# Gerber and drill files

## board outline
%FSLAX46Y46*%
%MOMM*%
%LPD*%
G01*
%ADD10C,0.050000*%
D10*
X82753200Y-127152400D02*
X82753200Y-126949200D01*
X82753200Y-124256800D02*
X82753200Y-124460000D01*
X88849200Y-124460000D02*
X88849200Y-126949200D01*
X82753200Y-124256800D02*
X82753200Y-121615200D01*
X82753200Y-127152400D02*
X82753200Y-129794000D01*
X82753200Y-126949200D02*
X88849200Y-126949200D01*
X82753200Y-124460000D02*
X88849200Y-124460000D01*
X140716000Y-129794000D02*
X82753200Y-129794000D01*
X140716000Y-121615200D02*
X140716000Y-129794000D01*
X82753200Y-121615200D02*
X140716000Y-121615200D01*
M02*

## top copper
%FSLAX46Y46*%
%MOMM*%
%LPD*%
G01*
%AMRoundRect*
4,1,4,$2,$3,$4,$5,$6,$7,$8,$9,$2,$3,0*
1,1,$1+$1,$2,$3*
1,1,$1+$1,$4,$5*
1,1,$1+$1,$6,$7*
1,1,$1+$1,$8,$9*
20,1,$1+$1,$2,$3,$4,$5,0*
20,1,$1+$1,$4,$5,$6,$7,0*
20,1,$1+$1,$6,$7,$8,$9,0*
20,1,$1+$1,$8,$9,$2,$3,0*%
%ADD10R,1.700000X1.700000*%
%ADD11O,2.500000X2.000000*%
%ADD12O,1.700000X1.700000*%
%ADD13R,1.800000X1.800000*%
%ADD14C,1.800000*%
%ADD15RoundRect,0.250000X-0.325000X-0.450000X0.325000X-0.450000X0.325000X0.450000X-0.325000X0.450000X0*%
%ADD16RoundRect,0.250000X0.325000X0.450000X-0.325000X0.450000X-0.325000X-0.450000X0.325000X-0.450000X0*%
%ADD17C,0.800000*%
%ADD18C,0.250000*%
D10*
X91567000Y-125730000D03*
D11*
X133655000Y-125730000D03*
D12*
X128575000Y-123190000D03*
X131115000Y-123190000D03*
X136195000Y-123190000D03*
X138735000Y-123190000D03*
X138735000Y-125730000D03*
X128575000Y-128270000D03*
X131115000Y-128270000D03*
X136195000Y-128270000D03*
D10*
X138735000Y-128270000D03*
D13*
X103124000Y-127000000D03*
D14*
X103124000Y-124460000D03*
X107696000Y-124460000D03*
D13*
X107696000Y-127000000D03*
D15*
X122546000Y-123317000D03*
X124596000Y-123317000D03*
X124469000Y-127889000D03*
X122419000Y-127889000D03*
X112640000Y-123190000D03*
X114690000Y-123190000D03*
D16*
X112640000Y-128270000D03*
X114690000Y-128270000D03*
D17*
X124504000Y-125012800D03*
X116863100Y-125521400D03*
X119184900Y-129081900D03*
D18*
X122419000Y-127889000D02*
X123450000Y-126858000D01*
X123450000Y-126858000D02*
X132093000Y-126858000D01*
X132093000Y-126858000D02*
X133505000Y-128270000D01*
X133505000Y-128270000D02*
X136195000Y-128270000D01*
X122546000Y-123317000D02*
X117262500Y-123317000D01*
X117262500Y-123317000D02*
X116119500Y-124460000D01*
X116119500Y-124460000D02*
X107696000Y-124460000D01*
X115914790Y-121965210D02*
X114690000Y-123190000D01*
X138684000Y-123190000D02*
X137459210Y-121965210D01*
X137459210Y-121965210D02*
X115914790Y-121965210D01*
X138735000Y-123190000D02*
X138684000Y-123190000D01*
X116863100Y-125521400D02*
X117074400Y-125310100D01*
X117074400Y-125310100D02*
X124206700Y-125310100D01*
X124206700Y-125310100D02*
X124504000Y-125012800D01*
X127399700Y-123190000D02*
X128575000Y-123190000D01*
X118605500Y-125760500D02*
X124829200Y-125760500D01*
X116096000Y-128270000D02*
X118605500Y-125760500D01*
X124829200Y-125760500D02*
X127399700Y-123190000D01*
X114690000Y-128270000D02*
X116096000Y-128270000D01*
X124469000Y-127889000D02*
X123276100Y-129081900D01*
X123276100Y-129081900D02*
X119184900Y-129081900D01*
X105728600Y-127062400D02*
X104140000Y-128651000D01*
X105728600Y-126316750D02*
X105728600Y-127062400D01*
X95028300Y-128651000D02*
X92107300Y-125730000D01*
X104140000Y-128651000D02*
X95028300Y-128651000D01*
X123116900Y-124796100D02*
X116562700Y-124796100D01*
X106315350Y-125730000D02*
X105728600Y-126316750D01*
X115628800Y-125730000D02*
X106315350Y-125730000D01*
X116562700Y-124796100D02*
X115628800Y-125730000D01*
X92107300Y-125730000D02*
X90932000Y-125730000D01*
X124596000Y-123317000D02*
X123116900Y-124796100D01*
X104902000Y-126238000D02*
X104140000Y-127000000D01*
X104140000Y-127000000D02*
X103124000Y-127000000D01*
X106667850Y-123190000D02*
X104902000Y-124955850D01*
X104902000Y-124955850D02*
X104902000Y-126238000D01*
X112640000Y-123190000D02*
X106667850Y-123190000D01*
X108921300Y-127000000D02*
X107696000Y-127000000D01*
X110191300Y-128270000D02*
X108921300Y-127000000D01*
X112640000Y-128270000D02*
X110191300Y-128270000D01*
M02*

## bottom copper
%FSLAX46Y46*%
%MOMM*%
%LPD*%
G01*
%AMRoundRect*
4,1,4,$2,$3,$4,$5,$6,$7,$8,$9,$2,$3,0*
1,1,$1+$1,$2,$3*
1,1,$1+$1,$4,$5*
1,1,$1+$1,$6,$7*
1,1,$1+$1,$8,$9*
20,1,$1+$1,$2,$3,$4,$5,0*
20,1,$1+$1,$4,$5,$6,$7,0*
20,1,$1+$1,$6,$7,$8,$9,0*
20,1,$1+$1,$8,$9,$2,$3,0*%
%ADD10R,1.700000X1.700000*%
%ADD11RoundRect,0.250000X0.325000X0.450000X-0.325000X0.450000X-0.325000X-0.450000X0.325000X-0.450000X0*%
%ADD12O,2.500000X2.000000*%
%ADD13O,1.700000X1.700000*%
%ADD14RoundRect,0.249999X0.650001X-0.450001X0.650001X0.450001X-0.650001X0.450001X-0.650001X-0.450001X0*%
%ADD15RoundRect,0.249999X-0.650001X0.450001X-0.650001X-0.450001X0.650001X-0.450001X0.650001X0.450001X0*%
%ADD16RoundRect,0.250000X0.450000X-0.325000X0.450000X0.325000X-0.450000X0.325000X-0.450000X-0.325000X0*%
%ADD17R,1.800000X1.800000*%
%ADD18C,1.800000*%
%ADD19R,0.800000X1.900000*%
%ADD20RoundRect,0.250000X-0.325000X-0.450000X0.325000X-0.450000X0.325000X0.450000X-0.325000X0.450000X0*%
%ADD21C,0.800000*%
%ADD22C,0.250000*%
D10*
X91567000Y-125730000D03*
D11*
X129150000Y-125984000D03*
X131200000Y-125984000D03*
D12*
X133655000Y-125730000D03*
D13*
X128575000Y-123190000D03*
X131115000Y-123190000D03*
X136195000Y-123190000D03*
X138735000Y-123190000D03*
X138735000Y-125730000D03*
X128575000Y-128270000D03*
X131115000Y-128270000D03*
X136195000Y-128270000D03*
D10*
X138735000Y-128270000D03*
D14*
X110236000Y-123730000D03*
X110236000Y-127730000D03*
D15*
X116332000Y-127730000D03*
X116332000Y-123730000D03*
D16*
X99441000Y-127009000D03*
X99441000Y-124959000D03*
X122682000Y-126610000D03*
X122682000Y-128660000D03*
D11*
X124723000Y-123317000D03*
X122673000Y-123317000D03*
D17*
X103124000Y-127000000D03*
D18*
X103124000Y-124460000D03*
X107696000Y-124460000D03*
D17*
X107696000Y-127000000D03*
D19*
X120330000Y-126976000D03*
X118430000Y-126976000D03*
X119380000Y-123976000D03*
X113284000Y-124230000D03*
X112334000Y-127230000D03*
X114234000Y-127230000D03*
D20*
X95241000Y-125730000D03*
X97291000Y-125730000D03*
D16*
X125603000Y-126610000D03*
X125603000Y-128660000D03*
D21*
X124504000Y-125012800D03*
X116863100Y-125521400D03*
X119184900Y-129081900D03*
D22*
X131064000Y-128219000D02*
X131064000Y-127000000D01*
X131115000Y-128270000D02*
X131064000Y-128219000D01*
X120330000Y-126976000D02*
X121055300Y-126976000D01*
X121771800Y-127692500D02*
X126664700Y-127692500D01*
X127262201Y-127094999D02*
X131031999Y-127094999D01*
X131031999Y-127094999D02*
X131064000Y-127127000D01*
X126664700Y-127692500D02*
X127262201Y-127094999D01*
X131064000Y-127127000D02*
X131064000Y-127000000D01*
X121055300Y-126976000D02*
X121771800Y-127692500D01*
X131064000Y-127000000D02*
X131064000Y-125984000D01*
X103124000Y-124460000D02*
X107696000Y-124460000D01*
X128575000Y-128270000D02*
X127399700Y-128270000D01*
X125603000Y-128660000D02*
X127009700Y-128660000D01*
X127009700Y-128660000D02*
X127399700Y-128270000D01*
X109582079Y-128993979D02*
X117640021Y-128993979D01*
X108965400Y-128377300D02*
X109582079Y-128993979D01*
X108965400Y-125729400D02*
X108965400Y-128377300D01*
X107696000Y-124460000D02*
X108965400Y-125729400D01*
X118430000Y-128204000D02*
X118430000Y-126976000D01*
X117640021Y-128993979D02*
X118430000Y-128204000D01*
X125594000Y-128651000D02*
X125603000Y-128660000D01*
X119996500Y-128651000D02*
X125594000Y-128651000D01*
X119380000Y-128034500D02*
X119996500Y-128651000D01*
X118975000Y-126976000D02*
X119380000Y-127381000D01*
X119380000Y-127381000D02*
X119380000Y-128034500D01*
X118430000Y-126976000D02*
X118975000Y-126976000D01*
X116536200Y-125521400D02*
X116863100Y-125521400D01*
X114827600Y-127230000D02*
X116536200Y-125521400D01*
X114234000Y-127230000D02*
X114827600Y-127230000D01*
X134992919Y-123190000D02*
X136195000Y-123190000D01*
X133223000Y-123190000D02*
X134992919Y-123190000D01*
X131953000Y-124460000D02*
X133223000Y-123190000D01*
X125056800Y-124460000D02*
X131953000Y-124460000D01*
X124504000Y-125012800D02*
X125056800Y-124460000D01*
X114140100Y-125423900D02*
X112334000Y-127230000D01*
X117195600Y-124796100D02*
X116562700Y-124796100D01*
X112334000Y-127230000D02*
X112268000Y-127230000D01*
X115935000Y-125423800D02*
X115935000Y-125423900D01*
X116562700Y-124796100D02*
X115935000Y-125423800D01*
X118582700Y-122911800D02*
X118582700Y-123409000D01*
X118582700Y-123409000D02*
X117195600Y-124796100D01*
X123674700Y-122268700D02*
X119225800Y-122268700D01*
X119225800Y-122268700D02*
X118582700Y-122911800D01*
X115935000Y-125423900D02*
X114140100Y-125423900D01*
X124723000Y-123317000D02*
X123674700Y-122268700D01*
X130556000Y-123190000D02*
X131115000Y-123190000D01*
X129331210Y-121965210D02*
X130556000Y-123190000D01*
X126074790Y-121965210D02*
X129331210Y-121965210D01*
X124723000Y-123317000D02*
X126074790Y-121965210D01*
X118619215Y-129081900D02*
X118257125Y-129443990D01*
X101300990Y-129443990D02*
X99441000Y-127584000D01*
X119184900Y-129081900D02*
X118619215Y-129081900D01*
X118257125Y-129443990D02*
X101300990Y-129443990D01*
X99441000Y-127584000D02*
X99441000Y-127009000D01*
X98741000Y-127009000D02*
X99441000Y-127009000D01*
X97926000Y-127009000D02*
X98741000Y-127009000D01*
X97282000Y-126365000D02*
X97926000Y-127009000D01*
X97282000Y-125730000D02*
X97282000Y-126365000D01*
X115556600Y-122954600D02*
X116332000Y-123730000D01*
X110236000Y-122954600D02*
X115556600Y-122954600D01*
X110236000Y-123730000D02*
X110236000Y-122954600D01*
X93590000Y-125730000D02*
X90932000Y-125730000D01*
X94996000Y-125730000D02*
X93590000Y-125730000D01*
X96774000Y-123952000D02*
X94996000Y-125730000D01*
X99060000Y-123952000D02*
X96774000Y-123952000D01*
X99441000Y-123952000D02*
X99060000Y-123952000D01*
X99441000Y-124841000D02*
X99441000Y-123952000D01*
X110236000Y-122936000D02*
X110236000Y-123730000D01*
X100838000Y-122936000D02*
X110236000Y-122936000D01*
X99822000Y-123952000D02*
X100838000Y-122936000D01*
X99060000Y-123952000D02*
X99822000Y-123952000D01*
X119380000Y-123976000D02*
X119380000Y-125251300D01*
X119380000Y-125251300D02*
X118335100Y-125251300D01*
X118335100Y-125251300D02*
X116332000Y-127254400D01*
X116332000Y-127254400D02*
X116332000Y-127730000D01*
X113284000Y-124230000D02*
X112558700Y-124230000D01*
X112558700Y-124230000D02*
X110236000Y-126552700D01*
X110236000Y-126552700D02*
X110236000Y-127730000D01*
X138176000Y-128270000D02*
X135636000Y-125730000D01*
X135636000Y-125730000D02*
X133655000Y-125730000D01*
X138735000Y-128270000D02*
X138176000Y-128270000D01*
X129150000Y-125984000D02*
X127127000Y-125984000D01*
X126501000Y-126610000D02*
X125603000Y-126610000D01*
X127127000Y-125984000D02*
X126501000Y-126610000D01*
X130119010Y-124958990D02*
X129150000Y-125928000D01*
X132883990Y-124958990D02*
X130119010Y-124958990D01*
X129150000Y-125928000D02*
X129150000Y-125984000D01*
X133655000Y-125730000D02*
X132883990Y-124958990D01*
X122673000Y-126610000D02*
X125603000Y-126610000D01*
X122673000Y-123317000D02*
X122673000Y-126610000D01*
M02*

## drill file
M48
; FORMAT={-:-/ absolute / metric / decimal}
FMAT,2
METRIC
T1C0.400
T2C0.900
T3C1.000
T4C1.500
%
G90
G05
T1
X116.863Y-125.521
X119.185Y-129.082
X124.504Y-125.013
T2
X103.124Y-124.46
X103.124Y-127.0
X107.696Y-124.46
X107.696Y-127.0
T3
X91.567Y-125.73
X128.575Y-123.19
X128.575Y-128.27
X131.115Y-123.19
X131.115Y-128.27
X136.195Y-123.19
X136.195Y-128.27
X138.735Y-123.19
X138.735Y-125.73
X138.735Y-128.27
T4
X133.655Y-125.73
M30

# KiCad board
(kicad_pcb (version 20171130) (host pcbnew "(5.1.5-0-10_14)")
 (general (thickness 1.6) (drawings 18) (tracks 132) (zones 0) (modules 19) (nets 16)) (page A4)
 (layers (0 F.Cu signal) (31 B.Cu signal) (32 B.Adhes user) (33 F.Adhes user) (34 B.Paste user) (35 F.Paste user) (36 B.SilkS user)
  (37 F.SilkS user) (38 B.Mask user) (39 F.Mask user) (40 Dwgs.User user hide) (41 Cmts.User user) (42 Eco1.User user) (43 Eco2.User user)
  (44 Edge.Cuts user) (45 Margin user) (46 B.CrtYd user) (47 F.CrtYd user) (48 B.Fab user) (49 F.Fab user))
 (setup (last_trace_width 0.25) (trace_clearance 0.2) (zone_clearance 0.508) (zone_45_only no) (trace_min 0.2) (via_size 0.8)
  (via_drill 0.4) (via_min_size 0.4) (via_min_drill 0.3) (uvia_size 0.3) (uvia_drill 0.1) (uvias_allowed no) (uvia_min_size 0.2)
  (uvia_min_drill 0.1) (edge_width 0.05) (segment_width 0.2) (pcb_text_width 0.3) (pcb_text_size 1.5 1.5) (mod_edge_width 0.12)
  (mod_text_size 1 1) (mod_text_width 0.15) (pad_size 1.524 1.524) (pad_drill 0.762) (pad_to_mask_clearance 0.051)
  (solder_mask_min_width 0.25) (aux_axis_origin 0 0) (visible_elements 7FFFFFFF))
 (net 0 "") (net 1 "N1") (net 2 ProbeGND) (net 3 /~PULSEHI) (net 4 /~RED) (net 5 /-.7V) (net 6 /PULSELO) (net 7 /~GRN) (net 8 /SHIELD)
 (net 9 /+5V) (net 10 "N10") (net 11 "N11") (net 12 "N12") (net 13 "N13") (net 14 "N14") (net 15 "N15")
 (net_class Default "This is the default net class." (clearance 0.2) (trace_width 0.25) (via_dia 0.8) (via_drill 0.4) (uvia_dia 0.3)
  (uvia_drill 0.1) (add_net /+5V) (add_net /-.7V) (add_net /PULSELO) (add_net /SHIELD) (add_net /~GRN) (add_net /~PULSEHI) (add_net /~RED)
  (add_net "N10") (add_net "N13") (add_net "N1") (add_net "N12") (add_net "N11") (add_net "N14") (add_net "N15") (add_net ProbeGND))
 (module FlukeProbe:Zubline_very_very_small (layer F.Cu) (at 96.774 125.73 60)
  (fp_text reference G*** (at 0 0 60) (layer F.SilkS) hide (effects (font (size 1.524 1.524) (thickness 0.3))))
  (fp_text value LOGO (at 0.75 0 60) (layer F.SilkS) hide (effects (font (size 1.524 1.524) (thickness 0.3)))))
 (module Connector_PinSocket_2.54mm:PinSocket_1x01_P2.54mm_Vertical (layer F.Cu) (at 91.567 125.73)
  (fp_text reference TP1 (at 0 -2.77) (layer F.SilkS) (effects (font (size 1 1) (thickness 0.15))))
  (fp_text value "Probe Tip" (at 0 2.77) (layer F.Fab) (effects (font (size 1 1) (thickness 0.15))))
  (pad 1 thru_hole rect (at 0 0) (size 1.7 1.7) (drill 1) (layers *.Cu *.Mask) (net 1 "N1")))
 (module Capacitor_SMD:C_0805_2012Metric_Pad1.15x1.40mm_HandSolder (layer B.Cu) (at 130.175 125.984 180)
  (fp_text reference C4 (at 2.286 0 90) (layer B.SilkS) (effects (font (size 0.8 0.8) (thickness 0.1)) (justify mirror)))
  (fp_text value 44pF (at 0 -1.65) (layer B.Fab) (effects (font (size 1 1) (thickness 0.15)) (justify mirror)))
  (pad 2 smd roundrect (at 1.025 0 180) (size 1.15 1.4) (layers B.Cu B.Paste B.Mask) (roundrect_rratio 0.217391) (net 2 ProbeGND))
  (pad 1 smd roundrect (at -1.025 0 180) (size 1.15 1.4) (layers B.Cu B.Paste B.Mask) (roundrect_rratio 0.217391) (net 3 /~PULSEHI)))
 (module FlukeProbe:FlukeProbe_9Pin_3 (layer B.Cu) (at 138.735 128.27 90)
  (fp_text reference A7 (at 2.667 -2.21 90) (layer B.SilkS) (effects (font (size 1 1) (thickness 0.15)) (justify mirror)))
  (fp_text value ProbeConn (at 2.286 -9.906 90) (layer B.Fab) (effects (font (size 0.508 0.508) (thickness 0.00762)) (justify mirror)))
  (pad 10 thru_hole oval (at 2.54 -5.08 90) (size 2 2.5) (drill 1.5) (layers *.Cu *.Mask) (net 2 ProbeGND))
  (pad 9 thru_hole oval (at 5.08 -10.16 90) (size 1.7 1.7) (drill 1) (layers *.Cu *.Mask) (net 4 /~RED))
  (pad 8 thru_hole oval (at 5.08 -7.62 90) (size 1.7 1.7) (drill 1) (layers *.Cu *.Mask) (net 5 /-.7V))
  (pad 7 thru_hole oval (at 5.08 -2.54 90) (size 1.7 1.7) (drill 1) (layers *.Cu *.Mask) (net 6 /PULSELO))
  (pad 6 thru_hole oval (at 5.08 0 90) (size 1.7 1.7) (drill 1) (layers *.Cu *.Mask) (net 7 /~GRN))
  (pad 5 thru_hole oval (at 2.54 0 90) (size 1.7 1.7) (drill 1) (layers *.Cu *.Mask) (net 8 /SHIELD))
  (pad 4 thru_hole oval (at 0 -10.16 90) (size 1.7 1.7) (drill 1) (layers *.Cu *.Mask) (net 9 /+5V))
  (pad 3 thru_hole oval (at 0 -7.62 90) (size 1.7 1.7) (drill 1) (layers *.Cu *.Mask) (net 3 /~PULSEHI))
  (pad 2 thru_hole oval (at 0 -2.54 90) (size 1.7 1.7) (drill 1) (layers *.Cu *.Mask) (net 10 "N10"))
  (pad 1 thru_hole rect (at 0 0 90) (size 1.7 1.7) (drill 1) (layers *.Cu *.Mask) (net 2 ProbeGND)))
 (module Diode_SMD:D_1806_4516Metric (layer B.Cu) (at 110.236 125.73 90)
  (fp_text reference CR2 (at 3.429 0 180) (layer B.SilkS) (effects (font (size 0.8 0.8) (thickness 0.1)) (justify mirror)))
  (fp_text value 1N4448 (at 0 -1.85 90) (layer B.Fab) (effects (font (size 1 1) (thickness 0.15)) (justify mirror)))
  (pad 2 smd roundrect (at 2 0 90) (size 1.4 1.8) (layers B.Cu B.Paste B.Mask) (roundrect_rratio 0.178571) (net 1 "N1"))
  (pad 1 smd roundrect (at -2 0 90) (size 1.4 1.8) (layers B.Cu B.Paste B.Mask) (roundrect_rratio 0.178571) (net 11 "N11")))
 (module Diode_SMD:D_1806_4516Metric (layer B.Cu) (at 116.332 125.73 270)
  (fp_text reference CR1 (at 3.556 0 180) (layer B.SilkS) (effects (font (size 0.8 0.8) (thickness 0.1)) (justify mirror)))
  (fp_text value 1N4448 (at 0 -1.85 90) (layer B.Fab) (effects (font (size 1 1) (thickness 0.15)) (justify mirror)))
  (pad 2 smd roundrect (at 2 0 270) (size 1.4 1.8) (layers B.Cu B.Paste B.Mask) (roundrect_rratio 0.178571) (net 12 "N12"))
  (pad 1 smd roundrect (at -2 0 270) (size 1.4 1.8) (layers B.Cu B.Paste B.Mask) (roundrect_rratio 0.178571) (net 1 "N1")))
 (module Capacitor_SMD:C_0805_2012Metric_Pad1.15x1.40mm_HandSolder (layer B.Cu) (at 99.441 125.984 90)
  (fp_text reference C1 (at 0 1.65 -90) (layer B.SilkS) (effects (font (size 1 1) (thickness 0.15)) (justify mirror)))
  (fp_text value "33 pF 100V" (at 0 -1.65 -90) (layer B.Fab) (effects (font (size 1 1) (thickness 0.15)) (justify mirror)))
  (pad 1 smd roundrect (at -1.025 0 90) (size 1.15 1.4) (layers B.Cu B.Paste B.Mask) (roundrect_rratio 0.217391) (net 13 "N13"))
  (pad 2 smd roundrect (at 1.025 0 90) (size 1.15 1.4) (layers B.Cu B.Paste B.Mask) (roundrect_rratio 0.217391) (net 1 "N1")))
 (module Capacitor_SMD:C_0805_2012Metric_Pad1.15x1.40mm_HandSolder (layer B.Cu) (at 122.682 127.635 90)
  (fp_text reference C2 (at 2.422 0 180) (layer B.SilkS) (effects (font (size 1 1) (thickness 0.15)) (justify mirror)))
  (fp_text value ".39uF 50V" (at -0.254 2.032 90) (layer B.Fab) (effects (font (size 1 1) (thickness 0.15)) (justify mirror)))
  (pad 2 smd roundrect (at 1.025 0 90) (size 1.15 1.4) (layers B.Cu B.Paste B.Mask) (roundrect_rratio 0.217391) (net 2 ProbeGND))
  (pad 1 smd roundrect (at -1.025 0 90) (size 1.15 1.4) (layers B.Cu B.Paste B.Mask) (roundrect_rratio 0.217391) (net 9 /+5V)))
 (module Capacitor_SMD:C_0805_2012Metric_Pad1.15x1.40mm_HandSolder (layer B.Cu) (at 123.698 123.317 180)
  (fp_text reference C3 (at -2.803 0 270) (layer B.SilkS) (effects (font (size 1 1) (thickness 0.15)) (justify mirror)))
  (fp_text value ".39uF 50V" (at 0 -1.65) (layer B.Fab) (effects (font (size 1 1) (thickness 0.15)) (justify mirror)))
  (pad 1 smd roundrect (at -1.025 0 180) (size 1.15 1.4) (layers B.Cu B.Paste B.Mask) (roundrect_rratio 0.217391) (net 5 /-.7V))
  (pad 2 smd roundrect (at 1.025 0 180) (size 1.15 1.4) (layers B.Cu B.Paste B.Mask) (roundrect_rratio 0.217391) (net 2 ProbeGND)))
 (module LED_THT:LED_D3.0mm (layer F.Cu) (at 103.124 127 90)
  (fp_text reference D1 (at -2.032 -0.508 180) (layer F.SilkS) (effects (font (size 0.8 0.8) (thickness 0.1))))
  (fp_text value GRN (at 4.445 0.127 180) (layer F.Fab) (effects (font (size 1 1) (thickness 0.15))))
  (pad 1 thru_hole rect (at 0 0 90) (size 1.8 1.8) (drill 0.9) (layers *.Cu *.Mask) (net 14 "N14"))
  (pad 2 thru_hole circle (at 2.54 0 90) (size 1.8 1.8) (drill 0.9) (layers *.Cu *.Mask) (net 9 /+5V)))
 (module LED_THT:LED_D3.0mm (layer F.Cu) (at 107.696 127 90)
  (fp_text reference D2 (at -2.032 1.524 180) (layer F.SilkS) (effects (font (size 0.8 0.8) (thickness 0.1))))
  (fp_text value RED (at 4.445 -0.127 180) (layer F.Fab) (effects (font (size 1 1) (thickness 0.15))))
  (pad 2 thru_hole circle (at 2.54 0 90) (size 1.8 1.8) (drill 0.9) (layers *.Cu *.Mask) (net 9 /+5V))
  (pad 1 thru_hole rect (at 0 0 90) (size 1.8 1.8) (drill 0.9) (layers *.Cu *.Mask) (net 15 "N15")))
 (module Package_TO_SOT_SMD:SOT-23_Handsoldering (layer B.Cu) (at 119.38 125.476 90)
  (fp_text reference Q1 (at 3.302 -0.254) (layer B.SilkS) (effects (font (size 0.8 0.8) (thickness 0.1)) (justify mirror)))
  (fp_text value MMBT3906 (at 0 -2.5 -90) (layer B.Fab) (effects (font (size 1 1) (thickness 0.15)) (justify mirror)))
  (pad 1 smd rect (at -1.5 0.95 90) (size 1.9 0.8) (layers B.Cu B.Paste B.Mask) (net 3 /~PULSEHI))
  (pad 2 smd rect (at -1.5 -0.95 90) (size 1.9 0.8) (layers B.Cu B.Paste B.Mask) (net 9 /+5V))
  (pad 3 smd rect (at 1.5 0 90) (size 1.9 0.8) (layers B.Cu B.Paste B.Mask) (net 12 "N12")))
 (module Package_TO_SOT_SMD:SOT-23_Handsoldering (layer B.Cu) (at 113.284 125.73 90)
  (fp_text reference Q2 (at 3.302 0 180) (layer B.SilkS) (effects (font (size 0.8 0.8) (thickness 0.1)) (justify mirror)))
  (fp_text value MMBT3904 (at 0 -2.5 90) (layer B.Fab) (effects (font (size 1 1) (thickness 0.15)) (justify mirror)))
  (pad 3 smd rect (at 1.5 0 90) (size 1.9 0.8) (layers B.Cu B.Paste B.Mask) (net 11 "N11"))
  (pad 2 smd rect (at -1.5 -0.95 90) (size 1.9 0.8) (layers B.Cu B.Paste B.Mask) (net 5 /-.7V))
  (pad 1 smd rect (at -1.5 0.95 90) (size 1.9 0.8) (layers B.Cu B.Paste B.Mask) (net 6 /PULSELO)))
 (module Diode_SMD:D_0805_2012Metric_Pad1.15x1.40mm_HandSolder (layer F.Cu) (at 123.571 123.317)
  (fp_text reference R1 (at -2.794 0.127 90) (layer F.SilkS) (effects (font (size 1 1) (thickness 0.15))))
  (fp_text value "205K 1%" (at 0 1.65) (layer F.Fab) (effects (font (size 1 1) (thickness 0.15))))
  (pad 1 smd roundrect (at -1.025 0) (size 1.15 1.4) (layers F.Cu F.Paste F.Mask) (roundrect_rratio 0.217391) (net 9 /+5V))
  (pad 2 smd roundrect (at 1.025 0) (size 1.15 1.4) (layers F.Cu F.Paste F.Mask) (roundrect_rratio 0.217391) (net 1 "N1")))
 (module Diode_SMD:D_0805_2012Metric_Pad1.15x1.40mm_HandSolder (layer F.Cu) (at 123.444 127.889)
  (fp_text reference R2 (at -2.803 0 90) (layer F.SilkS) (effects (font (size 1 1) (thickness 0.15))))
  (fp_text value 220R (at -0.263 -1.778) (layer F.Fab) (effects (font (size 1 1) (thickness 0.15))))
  (pad 2 smd roundrect (at 1.025 0) (size 1.15 1.4) (layers F.Cu F.Paste F.Mask) (roundrect_rratio 0.217391) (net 13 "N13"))
  (pad 1 smd roundrect (at -1.025 0) (size 1.15 1.4) (layers F.Cu F.Paste F.Mask) (roundrect_rratio 0.217391) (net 10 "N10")))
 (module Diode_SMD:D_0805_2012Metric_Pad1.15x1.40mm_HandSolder (layer B.Cu) (at 96.266 125.73)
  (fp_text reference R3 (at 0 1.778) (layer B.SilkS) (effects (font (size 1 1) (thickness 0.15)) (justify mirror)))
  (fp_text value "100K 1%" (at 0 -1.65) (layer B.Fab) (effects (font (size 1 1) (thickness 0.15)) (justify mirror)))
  (pad 1 smd roundrect (at -1.025 0) (size 1.15 1.4) (layers B.Cu B.Paste B.Mask) (roundrect_rratio 0.217391) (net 1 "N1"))
  (pad 2 smd roundrect (at 1.025 0) (size 1.15 1.4) (layers B.Cu B.Paste B.Mask) (roundrect_rratio 0.217391) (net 13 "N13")))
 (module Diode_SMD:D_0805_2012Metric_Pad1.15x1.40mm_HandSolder (layer B.Cu) (at 125.603 127.635 90)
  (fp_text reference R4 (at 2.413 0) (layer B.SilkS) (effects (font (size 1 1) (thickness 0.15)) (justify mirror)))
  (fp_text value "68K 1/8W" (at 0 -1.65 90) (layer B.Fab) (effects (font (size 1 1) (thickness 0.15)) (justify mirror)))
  (pad 2 smd roundrect (at 1.025 0 90) (size 1.15 1.4) (layers B.Cu B.Paste B.Mask) (roundrect_rratio 0.217391) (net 2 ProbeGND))
  (pad 1 smd roundrect (at -1.025 0 90) (size 1.15 1.4) (layers B.Cu B.Paste B.Mask) (roundrect_rratio 0.217391) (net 9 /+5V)))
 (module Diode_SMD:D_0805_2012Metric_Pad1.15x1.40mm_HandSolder (layer F.Cu) (at 113.665 123.19)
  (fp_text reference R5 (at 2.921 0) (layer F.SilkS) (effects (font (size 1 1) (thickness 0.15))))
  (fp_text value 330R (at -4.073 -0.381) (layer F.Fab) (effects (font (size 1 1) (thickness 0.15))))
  (pad 1 smd roundrect (at -1.025 0) (size 1.15 1.4) (layers F.Cu F.Paste F.Mask) (roundrect_rratio 0.217391) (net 14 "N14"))
  (pad 2 smd roundrect (at 1.025 0) (size 1.15 1.4) (layers F.Cu F.Paste F.Mask) (roundrect_rratio 0.217391) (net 7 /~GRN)))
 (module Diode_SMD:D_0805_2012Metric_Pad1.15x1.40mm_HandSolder (layer F.Cu) (at 113.665 128.27 180)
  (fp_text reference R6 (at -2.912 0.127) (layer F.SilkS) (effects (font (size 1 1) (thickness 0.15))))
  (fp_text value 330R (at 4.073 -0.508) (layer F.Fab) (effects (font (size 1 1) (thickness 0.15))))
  (pad 2 smd roundrect (at 1.025 0 180) (size 1.15 1.4) (layers F.Cu F.Paste F.Mask) (roundrect_rratio 0.217391) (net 15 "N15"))
  (pad 1 smd roundrect (at -1.025 0 180) (size 1.15 1.4) (layers F.Cu F.Paste F.Mask) (roundrect_rratio 0.217391) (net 4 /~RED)))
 (gr_line (start 82.7532 127.1524) (end 82.7532 126.9492) (layer Edge.Cuts) (width 0.05))
 (gr_line (start 82.7532 124.2568) (end 82.7532 124.46) (layer Edge.Cuts) (width 0.05))
 (gr_line (start 88.8492 124.46) (end 88.8492 126.9492) (layer Edge.Cuts) (width 0.05))
 (gr_line (start 82.7532 124.2568) (end 82.7532 121.6152) (layer Edge.Cuts) (width 0.05))
 (gr_line (start 82.7532 127.1524) (end 82.7532 129.794) (layer Edge.Cuts) (width 0.05))
 (gr_line (start 82.7532 126.9492) (end 88.8492 126.9492) (layer Edge.Cuts) (width 0.05))
 (gr_line (start 82.7532 124.46) (end 88.8492 124.46) (layer Edge.Cuts) (width 0.05))
 (gr_line (start 140.716 129.794) (end 82.7532 129.794) (layer Edge.Cuts) (width 0.05))
 (gr_line (start 140.716 121.6152) (end 140.716 129.794) (layer Edge.Cuts) (width 0.05))
 (gr_line (start 82.7532 121.6152) (end 140.716 121.6152) (layer Edge.Cuts) (width 0.05))
 (segment (start 122.419 127.889) (end 123.45 126.858) (width 0.25) (layer F.Cu) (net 10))
 (segment (start 123.45 126.858) (end 132.093 126.858) (width 0.25) (layer F.Cu) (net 10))
 (segment (start 132.093 126.858) (end 133.505 128.27) (width 0.25) (layer F.Cu) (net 10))
 (segment (start 133.505 128.27) (end 136.195 128.27) (width 0.25) (layer F.Cu) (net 10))
 (segment (start 131.064 128.219) (end 131.064 127) (width 0.25) (layer B.Cu) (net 3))
 (segment (start 131.115 128.27) (end 131.064 128.219) (width 0.25) (layer B.Cu) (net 3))
 (segment (start 120.33 126.976) (end 121.0553 126.976) (width 0.25) (layer B.Cu) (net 3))
 (segment (start 121.7718 127.6925) (end 126.6647 127.6925) (width 0.25) (layer B.Cu) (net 3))
 (segment (start 127.262201 127.094999) (end 131.031999 127.094999) (width 0.25) (layer B.Cu) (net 3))
 (segment (start 131.031999 127.094999) (end 131.064 127.127) (width 0.25) (layer B.Cu) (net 3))
 (segment (start 126.6647 127.6925) (end 127.262201 127.094999) (width 0.25) (layer B.Cu) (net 3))
 (segment (start 131.064 127.127) (end 131.064 127) (width 0.25) (layer B.Cu) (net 3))
 (segment (start 121.0553 126.976) (end 121.7718 127.6925) (width 0.25) (layer B.Cu) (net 3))
 (segment (start 131.064 127) (end 131.064 125.984) (width 0.25) (layer B.Cu) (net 3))
 (segment (start 122.546 123.317) (end 117.2625 123.317) (width 0.25) (layer F.Cu) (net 9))
 (segment (start 117.2625 123.317) (end 116.1195 124.46) (width 0.25) (layer F.Cu) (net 9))
 (segment (start 116.1195 124.46) (end 107.696 124.46) (width 0.25) (layer F.Cu) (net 9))
 (segment (start 103.124 124.46) (end 107.696 124.46) (width 0.25) (layer B.Cu) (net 9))
 (segment (start 128.575 128.27) (end 127.3997 128.27) (width 0.25) (layer B.Cu) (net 9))
 (segment (start 125.603 128.66) (end 127.0097 128.66) (width 0.25) (layer B.Cu) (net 9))
 (segment (start 127.0097 128.66) (end 127.3997 128.27) (width 0.25) (layer B.Cu) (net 9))
 (segment (start 109.582079 128.993979) (end 117.640021 128.993979) (width 0.25) (layer B.Cu) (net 9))
 (segment (start 108.9654 128.3773) (end 109.582079 128.993979) (width 0.25) (layer B.Cu) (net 9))
 (segment (start 108.9654 125.7294) (end 108.9654 128.3773) (width 0.25) (layer B.Cu) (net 9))
 (segment (start 107.696 124.46) (end 108.9654 125.7294) (width 0.25) (layer B.Cu) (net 9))
 (segment (start 118.43 128.204) (end 118.43 126.976) (width 0.25) (layer B.Cu) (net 9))
 (segment (start 117.640021 128.993979) (end 118.43 128.204) (width 0.25) (layer B.Cu) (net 9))
 (segment (start 125.594 128.651) (end 125.603 128.66) (width 0.25) (layer B.Cu) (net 9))
 (segment (start 119.9965 128.651) (end 125.594 128.651) (width 0.25) (layer B.Cu) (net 9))
 (segment (start 119.38 128.0345) (end 119.9965 128.651) (width 0.25) (layer B.Cu) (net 9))
 (segment (start 118.975 126.976) (end 119.38 127.381) (width 0.25) (layer B.Cu) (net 9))
 (segment (start 119.38 127.381) (end 119.38 128.0345) (width 0.25) (layer B.Cu) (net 9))
 (segment (start 118.43 126.976) (end 118.975 126.976) (width 0.25) (layer B.Cu) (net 9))
 (segment (start 115.91479 121.96521) (end 114.69 123.19) (width 0.25) (layer F.Cu) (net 7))
 (segment (start 138.684 123.19) (end 137.45921 121.96521) (width 0.25) (layer F.Cu) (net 7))
 (segment (start 137.45921 121.96521) (end 115.91479 121.96521) (width 0.25) (layer F.Cu) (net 7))
 (segment (start 138.735 123.19) (end 138.684 123.19) (width 0.25) (layer F.Cu) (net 7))
 (segment (start 116.8631 125.5214) (end 117.0744 125.3101) (width 0.25) (layer F.Cu) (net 6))
 (segment (start 117.0744 125.3101) (end 124.2067 125.3101) (width 0.25) (layer F.Cu) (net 6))
 (segment (start 124.2067 125.3101) (end 124.504 125.0128) (width 0.25) (layer F.Cu) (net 6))
 (via (at 124.504 125.0128) (size 0.8) (layers F.Cu B.Cu) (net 6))
 (via (at 116.8631 125.5214) (size 0.8) (layers F.Cu B.Cu) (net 6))
 (segment (start 116.5362 125.5214) (end 116.8631 125.5214) (width 0.25) (layer B.Cu) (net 6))
 (segment (start 114.8276 127.23) (end 116.5362 125.5214) (width 0.25) (layer B.Cu) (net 6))
 (segment (start 114.234 127.23) (end 114.8276 127.23) (width 0.25) (layer B.Cu) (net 6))
 (segment (start 134.992919 123.19) (end 136.195 123.19) (width 0.25) (layer B.Cu) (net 6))
 (segment (start 133.223 123.19) (end 134.992919 123.19) (width 0.25) (layer B.Cu) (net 6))
 (segment (start 131.953 124.46) (end 133.223 123.19) (width 0.25) (layer B.Cu) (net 6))
 (segment (start 125.0568 124.46) (end 131.953 124.46) (width 0.25) (layer B.Cu) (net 6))
 (segment (start 124.504 125.0128) (end 125.0568 124.46) (width 0.25) (layer B.Cu) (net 6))
 (segment (start 114.1401 125.4239) (end 112.334 127.23) (width 0.25) (layer B.Cu) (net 5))
 (segment (start 117.1956 124.7961) (end 116.5627 124.7961) (width 0.25) (layer B.Cu) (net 5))
 (segment (start 112.334 127.23) (end 112.268 127.23) (width 0.25) (layer B.Cu) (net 5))
 (segment (start 115.935 125.4238) (end 115.935 125.4239) (width 0.25) (layer B.Cu) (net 5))
 (segment (start 116.5627 124.7961) (end 115.935 125.4238) (width 0.25) (layer B.Cu) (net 5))
 (segment (start 118.5827 122.9118) (end 118.5827 123.409) (width 0.25) (layer B.Cu) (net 5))
 (segment (start 118.5827 123.409) (end 117.1956 124.7961) (width 0.25) (layer B.Cu) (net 5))
 (segment (start 123.6747 122.2687) (end 119.2258 122.2687) (width 0.25) (layer B.Cu) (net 5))
 (segment (start 119.2258 122.2687) (end 118.5827 122.9118) (width 0.25) (layer B.Cu) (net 5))
 (segment (start 115.935 125.4239) (end 114.1401 125.4239) (width 0.25) (layer B.Cu) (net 5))
 (segment (start 124.723 123.317) (end 123.6747 122.2687) (width 0.25) (layer B.Cu) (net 5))
 (segment (start 130.556 123.19) (end 131.115 123.19) (width 0.25) (layer B.Cu) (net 5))
 (segment (start 129.33121 121.96521) (end 130.556 123.19) (width 0.25) (layer B.Cu) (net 5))
 (segment (start 126.07479 121.96521) (end 129.33121 121.96521) (width 0.25) (layer B.Cu) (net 5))
 (segment (start 124.723 123.317) (end 126.07479 121.96521) (width 0.25) (layer B.Cu) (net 5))
 (segment (start 127.3997 123.19) (end 128.575 123.19) (width 0.25) (layer F.Cu) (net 4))
 (segment (start 118.6055 125.7605) (end 124.8292 125.7605) (width 0.25) (layer F.Cu) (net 4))
 (segment (start 116.096 128.27) (end 118.6055 125.7605) (width 0.25) (layer F.Cu) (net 4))
 (segment (start 124.8292 125.7605) (end 127.3997 123.19) (width 0.25) (layer F.Cu) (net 4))
 (segment (start 114.69 128.27) (end 116.096 128.27) (width 0.25) (layer F.Cu) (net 4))
 (segment (start 124.469 127.889) (end 123.2761 129.0819) (width 0.25) (layer F.Cu) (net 13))
 (via (at 119.1849 129.0819) (size 0.8) (layers F.Cu B.Cu) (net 13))
 (segment (start 123.2761 129.0819) (end 119.1849 129.0819) (width 0.25) (layer F.Cu) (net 13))
 (segment (start 118.619215 129.0819) (end 118.257125 129.44399) (width 0.25) (layer B.Cu) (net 13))
 (segment (start 101.30099 129.44399) (end 99.441 127.584) (width 0.25) (layer B.Cu) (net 13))
 (segment (start 119.1849 129.0819) (end 118.619215 129.0819) (width 0.25) (layer B.Cu) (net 13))
 (segment (start 118.257125 129.44399) (end 101.30099 129.44399) (width 0.25) (layer B.Cu) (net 13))
 (segment (start 99.441 127.584) (end 99.441 127.009) (width 0.25) (layer B.Cu) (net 13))
 (segment (start 98.741 127.009) (end 99.441 127.009) (width 0.25) (layer B.Cu) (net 13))
 (segment (start 97.926 127.009) (end 98.741 127.009) (width 0.25) (layer B.Cu) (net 13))
 (segment (start 97.282 126.365) (end 97.926 127.009) (width 0.25) (layer B.Cu) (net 13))
 (segment (start 97.282 125.73) (end 97.282 126.365) (width 0.25) (layer B.Cu) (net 13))
 (segment (start 115.5566 122.9546) (end 116.332 123.73) (width 0.25) (layer B.Cu) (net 1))
 (segment (start 110.236 122.9546) (end 115.5566 122.9546) (width 0.25) (layer B.Cu) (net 1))
 (segment (start 110.236 123.73) (end 110.236 122.9546) (width 0.25) (layer B.Cu) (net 1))
 (segment (start 93.59 125.73) (end 90.932 125.73) (width 0.25) (layer B.Cu) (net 1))
 (segment (start 94.996 125.73) (end 93.59 125.73) (width 0.25) (layer B.Cu) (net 1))
 (segment (start 96.774 123.952) (end 94.996 125.73) (width 0.25) (layer B.Cu) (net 1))
 (segment (start 99.06 123.952) (end 96.774 123.952) (width 0.25) (layer B.Cu) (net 1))
 (segment (start 105.7286 127.0624) (end 104.14 128.651) (width 0.25) (layer F.Cu) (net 1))
 (segment (start 105.7286 126.31675) (end 105.7286 127.0624) (width 0.25) (layer F.Cu) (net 1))
 (segment (start 95.0283 128.651) (end 92.1073 125.73) (width 0.25) (layer F.Cu) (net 1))
 (segment (start 104.14 128.651) (end 95.0283 128.651) (width 0.25) (layer F.Cu) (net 1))
 (segment (start 123.1169 124.7961) (end 116.5627 124.7961) (width 0.25) (layer F.Cu) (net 1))
 (segment (start 106.31535 125.73) (end 105.7286 126.31675) (width 0.25) (layer F.Cu) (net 1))
 (segment (start 115.6288 125.73) (end 106.31535 125.73) (width 0.25) (layer F.Cu) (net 1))
 (segment (start 116.5627 124.7961) (end 115.6288 125.73) (width 0.25) (layer F.Cu) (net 1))
 (segment (start 92.1073 125.73) (end 90.932 125.73) (width 0.25) (layer F.Cu) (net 1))
 (segment (start 124.596 123.317) (end 123.1169 124.7961) (width 0.25) (layer F.Cu) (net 1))
 (segment (start 99.441 123.952) (end 99.06 123.952) (width 0.25) (layer B.Cu) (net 1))
 (segment (start 99.441 124.841) (end 99.441 123.952) (width 0.25) (layer B.Cu) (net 1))
 (segment (start 110.236 122.936) (end 110.236 123.73) (width 0.25) (layer B.Cu) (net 1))
 (segment (start 100.838 122.936) (end 110.236 122.936) (width 0.25) (layer B.Cu) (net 1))
 (segment (start 99.822 123.952) (end 100.838 122.936) (width 0.25) (layer B.Cu) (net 1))
 (segment (start 99.06 123.952) (end 99.822 123.952) (width 0.25) (layer B.Cu) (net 1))
 (segment (start 119.38 123.976) (end 119.38 125.2513) (width 0.25) (layer B.Cu) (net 12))
 (segment (start 119.38 125.2513) (end 118.3351 125.2513) (width 0.25) (layer B.Cu) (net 12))
 (segment (start 118.3351 125.2513) (end 116.332 127.2544) (width 0.25) (layer B.Cu) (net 12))
 (segment (start 116.332 127.2544) (end 116.332 127.73) (width 0.25) (layer B.Cu) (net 12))
 (segment (start 113.284 124.23) (end 112.5587 124.23) (width 0.25) (layer B.Cu) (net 11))
 (segment (start 112.5587 124.23) (end 110.236 126.5527) (width 0.25) (layer B.Cu) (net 11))
 (segment (start 110.236 126.5527) (end 110.236 127.73) (width 0.25) (layer B.Cu) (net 11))
 (segment (start 104.902 126.238) (end 104.14 127) (width 0.25) (layer F.Cu) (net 14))
 (segment (start 104.14 127) (end 103.124 127) (width 0.25) (layer F.Cu) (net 14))
 (segment (start 106.66785 123.19) (end 104.902 124.95585) (width 0.25) (layer F.Cu) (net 14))
 (segment (start 104.902 124.95585) (end 104.902 126.238) (width 0.25) (layer F.Cu) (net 14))
 (segment (start 112.64 123.19) (end 106.66785 123.19) (width 0.25) (layer F.Cu) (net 14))
 (segment (start 108.9213 127) (end 107.696 127) (width 0.25) (layer F.Cu) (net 15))
 (segment (start 110.1913 128.27) (end 108.9213 127) (width 0.25) (layer F.Cu) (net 15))
 (segment (start 112.64 128.27) (end 110.1913 128.27) (width 0.25) (layer F.Cu) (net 15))
 (segment (start 138.176 128.27) (end 135.636 125.73) (width 0.25) (layer B.Cu) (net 2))
 (segment (start 135.636 125.73) (end 133.655 125.73) (width 0.25) (layer B.Cu) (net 2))
 (segment (start 138.735 128.27) (end 138.176 128.27) (width 0.25) (layer B.Cu) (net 2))
 (segment (start 129.15 125.984) (end 127.127 125.984) (width 0.25) (layer B.Cu) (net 2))
 (segment (start 126.501 126.61) (end 125.603 126.61) (width 0.25) (layer B.Cu) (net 2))
 (segment (start 127.127 125.984) (end 126.501 126.61) (width 0.25) (layer B.Cu) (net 2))
 (segment (start 130.11901 124.95899) (end 129.15 125.928) (width 0.25) (layer B.Cu) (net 2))
 (segment (start 132.88399 124.95899) (end 130.11901 124.95899) (width 0.25) (layer B.Cu) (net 2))
 (segment (start 129.15 125.928) (end 129.15 125.984) (width 0.25) (layer B.Cu) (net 2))
 (segment (start 133.655 125.73) (end 132.88399 124.95899) (width 0.25) (layer B.Cu) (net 2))
 (segment (start 122.673 126.61) (end 125.603 126.61) (width 0.25) (layer B.Cu) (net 2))
 (segment (start 122.673 123.317) (end 122.673 126.61) (width 0.25) (layer B.Cu) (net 2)))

